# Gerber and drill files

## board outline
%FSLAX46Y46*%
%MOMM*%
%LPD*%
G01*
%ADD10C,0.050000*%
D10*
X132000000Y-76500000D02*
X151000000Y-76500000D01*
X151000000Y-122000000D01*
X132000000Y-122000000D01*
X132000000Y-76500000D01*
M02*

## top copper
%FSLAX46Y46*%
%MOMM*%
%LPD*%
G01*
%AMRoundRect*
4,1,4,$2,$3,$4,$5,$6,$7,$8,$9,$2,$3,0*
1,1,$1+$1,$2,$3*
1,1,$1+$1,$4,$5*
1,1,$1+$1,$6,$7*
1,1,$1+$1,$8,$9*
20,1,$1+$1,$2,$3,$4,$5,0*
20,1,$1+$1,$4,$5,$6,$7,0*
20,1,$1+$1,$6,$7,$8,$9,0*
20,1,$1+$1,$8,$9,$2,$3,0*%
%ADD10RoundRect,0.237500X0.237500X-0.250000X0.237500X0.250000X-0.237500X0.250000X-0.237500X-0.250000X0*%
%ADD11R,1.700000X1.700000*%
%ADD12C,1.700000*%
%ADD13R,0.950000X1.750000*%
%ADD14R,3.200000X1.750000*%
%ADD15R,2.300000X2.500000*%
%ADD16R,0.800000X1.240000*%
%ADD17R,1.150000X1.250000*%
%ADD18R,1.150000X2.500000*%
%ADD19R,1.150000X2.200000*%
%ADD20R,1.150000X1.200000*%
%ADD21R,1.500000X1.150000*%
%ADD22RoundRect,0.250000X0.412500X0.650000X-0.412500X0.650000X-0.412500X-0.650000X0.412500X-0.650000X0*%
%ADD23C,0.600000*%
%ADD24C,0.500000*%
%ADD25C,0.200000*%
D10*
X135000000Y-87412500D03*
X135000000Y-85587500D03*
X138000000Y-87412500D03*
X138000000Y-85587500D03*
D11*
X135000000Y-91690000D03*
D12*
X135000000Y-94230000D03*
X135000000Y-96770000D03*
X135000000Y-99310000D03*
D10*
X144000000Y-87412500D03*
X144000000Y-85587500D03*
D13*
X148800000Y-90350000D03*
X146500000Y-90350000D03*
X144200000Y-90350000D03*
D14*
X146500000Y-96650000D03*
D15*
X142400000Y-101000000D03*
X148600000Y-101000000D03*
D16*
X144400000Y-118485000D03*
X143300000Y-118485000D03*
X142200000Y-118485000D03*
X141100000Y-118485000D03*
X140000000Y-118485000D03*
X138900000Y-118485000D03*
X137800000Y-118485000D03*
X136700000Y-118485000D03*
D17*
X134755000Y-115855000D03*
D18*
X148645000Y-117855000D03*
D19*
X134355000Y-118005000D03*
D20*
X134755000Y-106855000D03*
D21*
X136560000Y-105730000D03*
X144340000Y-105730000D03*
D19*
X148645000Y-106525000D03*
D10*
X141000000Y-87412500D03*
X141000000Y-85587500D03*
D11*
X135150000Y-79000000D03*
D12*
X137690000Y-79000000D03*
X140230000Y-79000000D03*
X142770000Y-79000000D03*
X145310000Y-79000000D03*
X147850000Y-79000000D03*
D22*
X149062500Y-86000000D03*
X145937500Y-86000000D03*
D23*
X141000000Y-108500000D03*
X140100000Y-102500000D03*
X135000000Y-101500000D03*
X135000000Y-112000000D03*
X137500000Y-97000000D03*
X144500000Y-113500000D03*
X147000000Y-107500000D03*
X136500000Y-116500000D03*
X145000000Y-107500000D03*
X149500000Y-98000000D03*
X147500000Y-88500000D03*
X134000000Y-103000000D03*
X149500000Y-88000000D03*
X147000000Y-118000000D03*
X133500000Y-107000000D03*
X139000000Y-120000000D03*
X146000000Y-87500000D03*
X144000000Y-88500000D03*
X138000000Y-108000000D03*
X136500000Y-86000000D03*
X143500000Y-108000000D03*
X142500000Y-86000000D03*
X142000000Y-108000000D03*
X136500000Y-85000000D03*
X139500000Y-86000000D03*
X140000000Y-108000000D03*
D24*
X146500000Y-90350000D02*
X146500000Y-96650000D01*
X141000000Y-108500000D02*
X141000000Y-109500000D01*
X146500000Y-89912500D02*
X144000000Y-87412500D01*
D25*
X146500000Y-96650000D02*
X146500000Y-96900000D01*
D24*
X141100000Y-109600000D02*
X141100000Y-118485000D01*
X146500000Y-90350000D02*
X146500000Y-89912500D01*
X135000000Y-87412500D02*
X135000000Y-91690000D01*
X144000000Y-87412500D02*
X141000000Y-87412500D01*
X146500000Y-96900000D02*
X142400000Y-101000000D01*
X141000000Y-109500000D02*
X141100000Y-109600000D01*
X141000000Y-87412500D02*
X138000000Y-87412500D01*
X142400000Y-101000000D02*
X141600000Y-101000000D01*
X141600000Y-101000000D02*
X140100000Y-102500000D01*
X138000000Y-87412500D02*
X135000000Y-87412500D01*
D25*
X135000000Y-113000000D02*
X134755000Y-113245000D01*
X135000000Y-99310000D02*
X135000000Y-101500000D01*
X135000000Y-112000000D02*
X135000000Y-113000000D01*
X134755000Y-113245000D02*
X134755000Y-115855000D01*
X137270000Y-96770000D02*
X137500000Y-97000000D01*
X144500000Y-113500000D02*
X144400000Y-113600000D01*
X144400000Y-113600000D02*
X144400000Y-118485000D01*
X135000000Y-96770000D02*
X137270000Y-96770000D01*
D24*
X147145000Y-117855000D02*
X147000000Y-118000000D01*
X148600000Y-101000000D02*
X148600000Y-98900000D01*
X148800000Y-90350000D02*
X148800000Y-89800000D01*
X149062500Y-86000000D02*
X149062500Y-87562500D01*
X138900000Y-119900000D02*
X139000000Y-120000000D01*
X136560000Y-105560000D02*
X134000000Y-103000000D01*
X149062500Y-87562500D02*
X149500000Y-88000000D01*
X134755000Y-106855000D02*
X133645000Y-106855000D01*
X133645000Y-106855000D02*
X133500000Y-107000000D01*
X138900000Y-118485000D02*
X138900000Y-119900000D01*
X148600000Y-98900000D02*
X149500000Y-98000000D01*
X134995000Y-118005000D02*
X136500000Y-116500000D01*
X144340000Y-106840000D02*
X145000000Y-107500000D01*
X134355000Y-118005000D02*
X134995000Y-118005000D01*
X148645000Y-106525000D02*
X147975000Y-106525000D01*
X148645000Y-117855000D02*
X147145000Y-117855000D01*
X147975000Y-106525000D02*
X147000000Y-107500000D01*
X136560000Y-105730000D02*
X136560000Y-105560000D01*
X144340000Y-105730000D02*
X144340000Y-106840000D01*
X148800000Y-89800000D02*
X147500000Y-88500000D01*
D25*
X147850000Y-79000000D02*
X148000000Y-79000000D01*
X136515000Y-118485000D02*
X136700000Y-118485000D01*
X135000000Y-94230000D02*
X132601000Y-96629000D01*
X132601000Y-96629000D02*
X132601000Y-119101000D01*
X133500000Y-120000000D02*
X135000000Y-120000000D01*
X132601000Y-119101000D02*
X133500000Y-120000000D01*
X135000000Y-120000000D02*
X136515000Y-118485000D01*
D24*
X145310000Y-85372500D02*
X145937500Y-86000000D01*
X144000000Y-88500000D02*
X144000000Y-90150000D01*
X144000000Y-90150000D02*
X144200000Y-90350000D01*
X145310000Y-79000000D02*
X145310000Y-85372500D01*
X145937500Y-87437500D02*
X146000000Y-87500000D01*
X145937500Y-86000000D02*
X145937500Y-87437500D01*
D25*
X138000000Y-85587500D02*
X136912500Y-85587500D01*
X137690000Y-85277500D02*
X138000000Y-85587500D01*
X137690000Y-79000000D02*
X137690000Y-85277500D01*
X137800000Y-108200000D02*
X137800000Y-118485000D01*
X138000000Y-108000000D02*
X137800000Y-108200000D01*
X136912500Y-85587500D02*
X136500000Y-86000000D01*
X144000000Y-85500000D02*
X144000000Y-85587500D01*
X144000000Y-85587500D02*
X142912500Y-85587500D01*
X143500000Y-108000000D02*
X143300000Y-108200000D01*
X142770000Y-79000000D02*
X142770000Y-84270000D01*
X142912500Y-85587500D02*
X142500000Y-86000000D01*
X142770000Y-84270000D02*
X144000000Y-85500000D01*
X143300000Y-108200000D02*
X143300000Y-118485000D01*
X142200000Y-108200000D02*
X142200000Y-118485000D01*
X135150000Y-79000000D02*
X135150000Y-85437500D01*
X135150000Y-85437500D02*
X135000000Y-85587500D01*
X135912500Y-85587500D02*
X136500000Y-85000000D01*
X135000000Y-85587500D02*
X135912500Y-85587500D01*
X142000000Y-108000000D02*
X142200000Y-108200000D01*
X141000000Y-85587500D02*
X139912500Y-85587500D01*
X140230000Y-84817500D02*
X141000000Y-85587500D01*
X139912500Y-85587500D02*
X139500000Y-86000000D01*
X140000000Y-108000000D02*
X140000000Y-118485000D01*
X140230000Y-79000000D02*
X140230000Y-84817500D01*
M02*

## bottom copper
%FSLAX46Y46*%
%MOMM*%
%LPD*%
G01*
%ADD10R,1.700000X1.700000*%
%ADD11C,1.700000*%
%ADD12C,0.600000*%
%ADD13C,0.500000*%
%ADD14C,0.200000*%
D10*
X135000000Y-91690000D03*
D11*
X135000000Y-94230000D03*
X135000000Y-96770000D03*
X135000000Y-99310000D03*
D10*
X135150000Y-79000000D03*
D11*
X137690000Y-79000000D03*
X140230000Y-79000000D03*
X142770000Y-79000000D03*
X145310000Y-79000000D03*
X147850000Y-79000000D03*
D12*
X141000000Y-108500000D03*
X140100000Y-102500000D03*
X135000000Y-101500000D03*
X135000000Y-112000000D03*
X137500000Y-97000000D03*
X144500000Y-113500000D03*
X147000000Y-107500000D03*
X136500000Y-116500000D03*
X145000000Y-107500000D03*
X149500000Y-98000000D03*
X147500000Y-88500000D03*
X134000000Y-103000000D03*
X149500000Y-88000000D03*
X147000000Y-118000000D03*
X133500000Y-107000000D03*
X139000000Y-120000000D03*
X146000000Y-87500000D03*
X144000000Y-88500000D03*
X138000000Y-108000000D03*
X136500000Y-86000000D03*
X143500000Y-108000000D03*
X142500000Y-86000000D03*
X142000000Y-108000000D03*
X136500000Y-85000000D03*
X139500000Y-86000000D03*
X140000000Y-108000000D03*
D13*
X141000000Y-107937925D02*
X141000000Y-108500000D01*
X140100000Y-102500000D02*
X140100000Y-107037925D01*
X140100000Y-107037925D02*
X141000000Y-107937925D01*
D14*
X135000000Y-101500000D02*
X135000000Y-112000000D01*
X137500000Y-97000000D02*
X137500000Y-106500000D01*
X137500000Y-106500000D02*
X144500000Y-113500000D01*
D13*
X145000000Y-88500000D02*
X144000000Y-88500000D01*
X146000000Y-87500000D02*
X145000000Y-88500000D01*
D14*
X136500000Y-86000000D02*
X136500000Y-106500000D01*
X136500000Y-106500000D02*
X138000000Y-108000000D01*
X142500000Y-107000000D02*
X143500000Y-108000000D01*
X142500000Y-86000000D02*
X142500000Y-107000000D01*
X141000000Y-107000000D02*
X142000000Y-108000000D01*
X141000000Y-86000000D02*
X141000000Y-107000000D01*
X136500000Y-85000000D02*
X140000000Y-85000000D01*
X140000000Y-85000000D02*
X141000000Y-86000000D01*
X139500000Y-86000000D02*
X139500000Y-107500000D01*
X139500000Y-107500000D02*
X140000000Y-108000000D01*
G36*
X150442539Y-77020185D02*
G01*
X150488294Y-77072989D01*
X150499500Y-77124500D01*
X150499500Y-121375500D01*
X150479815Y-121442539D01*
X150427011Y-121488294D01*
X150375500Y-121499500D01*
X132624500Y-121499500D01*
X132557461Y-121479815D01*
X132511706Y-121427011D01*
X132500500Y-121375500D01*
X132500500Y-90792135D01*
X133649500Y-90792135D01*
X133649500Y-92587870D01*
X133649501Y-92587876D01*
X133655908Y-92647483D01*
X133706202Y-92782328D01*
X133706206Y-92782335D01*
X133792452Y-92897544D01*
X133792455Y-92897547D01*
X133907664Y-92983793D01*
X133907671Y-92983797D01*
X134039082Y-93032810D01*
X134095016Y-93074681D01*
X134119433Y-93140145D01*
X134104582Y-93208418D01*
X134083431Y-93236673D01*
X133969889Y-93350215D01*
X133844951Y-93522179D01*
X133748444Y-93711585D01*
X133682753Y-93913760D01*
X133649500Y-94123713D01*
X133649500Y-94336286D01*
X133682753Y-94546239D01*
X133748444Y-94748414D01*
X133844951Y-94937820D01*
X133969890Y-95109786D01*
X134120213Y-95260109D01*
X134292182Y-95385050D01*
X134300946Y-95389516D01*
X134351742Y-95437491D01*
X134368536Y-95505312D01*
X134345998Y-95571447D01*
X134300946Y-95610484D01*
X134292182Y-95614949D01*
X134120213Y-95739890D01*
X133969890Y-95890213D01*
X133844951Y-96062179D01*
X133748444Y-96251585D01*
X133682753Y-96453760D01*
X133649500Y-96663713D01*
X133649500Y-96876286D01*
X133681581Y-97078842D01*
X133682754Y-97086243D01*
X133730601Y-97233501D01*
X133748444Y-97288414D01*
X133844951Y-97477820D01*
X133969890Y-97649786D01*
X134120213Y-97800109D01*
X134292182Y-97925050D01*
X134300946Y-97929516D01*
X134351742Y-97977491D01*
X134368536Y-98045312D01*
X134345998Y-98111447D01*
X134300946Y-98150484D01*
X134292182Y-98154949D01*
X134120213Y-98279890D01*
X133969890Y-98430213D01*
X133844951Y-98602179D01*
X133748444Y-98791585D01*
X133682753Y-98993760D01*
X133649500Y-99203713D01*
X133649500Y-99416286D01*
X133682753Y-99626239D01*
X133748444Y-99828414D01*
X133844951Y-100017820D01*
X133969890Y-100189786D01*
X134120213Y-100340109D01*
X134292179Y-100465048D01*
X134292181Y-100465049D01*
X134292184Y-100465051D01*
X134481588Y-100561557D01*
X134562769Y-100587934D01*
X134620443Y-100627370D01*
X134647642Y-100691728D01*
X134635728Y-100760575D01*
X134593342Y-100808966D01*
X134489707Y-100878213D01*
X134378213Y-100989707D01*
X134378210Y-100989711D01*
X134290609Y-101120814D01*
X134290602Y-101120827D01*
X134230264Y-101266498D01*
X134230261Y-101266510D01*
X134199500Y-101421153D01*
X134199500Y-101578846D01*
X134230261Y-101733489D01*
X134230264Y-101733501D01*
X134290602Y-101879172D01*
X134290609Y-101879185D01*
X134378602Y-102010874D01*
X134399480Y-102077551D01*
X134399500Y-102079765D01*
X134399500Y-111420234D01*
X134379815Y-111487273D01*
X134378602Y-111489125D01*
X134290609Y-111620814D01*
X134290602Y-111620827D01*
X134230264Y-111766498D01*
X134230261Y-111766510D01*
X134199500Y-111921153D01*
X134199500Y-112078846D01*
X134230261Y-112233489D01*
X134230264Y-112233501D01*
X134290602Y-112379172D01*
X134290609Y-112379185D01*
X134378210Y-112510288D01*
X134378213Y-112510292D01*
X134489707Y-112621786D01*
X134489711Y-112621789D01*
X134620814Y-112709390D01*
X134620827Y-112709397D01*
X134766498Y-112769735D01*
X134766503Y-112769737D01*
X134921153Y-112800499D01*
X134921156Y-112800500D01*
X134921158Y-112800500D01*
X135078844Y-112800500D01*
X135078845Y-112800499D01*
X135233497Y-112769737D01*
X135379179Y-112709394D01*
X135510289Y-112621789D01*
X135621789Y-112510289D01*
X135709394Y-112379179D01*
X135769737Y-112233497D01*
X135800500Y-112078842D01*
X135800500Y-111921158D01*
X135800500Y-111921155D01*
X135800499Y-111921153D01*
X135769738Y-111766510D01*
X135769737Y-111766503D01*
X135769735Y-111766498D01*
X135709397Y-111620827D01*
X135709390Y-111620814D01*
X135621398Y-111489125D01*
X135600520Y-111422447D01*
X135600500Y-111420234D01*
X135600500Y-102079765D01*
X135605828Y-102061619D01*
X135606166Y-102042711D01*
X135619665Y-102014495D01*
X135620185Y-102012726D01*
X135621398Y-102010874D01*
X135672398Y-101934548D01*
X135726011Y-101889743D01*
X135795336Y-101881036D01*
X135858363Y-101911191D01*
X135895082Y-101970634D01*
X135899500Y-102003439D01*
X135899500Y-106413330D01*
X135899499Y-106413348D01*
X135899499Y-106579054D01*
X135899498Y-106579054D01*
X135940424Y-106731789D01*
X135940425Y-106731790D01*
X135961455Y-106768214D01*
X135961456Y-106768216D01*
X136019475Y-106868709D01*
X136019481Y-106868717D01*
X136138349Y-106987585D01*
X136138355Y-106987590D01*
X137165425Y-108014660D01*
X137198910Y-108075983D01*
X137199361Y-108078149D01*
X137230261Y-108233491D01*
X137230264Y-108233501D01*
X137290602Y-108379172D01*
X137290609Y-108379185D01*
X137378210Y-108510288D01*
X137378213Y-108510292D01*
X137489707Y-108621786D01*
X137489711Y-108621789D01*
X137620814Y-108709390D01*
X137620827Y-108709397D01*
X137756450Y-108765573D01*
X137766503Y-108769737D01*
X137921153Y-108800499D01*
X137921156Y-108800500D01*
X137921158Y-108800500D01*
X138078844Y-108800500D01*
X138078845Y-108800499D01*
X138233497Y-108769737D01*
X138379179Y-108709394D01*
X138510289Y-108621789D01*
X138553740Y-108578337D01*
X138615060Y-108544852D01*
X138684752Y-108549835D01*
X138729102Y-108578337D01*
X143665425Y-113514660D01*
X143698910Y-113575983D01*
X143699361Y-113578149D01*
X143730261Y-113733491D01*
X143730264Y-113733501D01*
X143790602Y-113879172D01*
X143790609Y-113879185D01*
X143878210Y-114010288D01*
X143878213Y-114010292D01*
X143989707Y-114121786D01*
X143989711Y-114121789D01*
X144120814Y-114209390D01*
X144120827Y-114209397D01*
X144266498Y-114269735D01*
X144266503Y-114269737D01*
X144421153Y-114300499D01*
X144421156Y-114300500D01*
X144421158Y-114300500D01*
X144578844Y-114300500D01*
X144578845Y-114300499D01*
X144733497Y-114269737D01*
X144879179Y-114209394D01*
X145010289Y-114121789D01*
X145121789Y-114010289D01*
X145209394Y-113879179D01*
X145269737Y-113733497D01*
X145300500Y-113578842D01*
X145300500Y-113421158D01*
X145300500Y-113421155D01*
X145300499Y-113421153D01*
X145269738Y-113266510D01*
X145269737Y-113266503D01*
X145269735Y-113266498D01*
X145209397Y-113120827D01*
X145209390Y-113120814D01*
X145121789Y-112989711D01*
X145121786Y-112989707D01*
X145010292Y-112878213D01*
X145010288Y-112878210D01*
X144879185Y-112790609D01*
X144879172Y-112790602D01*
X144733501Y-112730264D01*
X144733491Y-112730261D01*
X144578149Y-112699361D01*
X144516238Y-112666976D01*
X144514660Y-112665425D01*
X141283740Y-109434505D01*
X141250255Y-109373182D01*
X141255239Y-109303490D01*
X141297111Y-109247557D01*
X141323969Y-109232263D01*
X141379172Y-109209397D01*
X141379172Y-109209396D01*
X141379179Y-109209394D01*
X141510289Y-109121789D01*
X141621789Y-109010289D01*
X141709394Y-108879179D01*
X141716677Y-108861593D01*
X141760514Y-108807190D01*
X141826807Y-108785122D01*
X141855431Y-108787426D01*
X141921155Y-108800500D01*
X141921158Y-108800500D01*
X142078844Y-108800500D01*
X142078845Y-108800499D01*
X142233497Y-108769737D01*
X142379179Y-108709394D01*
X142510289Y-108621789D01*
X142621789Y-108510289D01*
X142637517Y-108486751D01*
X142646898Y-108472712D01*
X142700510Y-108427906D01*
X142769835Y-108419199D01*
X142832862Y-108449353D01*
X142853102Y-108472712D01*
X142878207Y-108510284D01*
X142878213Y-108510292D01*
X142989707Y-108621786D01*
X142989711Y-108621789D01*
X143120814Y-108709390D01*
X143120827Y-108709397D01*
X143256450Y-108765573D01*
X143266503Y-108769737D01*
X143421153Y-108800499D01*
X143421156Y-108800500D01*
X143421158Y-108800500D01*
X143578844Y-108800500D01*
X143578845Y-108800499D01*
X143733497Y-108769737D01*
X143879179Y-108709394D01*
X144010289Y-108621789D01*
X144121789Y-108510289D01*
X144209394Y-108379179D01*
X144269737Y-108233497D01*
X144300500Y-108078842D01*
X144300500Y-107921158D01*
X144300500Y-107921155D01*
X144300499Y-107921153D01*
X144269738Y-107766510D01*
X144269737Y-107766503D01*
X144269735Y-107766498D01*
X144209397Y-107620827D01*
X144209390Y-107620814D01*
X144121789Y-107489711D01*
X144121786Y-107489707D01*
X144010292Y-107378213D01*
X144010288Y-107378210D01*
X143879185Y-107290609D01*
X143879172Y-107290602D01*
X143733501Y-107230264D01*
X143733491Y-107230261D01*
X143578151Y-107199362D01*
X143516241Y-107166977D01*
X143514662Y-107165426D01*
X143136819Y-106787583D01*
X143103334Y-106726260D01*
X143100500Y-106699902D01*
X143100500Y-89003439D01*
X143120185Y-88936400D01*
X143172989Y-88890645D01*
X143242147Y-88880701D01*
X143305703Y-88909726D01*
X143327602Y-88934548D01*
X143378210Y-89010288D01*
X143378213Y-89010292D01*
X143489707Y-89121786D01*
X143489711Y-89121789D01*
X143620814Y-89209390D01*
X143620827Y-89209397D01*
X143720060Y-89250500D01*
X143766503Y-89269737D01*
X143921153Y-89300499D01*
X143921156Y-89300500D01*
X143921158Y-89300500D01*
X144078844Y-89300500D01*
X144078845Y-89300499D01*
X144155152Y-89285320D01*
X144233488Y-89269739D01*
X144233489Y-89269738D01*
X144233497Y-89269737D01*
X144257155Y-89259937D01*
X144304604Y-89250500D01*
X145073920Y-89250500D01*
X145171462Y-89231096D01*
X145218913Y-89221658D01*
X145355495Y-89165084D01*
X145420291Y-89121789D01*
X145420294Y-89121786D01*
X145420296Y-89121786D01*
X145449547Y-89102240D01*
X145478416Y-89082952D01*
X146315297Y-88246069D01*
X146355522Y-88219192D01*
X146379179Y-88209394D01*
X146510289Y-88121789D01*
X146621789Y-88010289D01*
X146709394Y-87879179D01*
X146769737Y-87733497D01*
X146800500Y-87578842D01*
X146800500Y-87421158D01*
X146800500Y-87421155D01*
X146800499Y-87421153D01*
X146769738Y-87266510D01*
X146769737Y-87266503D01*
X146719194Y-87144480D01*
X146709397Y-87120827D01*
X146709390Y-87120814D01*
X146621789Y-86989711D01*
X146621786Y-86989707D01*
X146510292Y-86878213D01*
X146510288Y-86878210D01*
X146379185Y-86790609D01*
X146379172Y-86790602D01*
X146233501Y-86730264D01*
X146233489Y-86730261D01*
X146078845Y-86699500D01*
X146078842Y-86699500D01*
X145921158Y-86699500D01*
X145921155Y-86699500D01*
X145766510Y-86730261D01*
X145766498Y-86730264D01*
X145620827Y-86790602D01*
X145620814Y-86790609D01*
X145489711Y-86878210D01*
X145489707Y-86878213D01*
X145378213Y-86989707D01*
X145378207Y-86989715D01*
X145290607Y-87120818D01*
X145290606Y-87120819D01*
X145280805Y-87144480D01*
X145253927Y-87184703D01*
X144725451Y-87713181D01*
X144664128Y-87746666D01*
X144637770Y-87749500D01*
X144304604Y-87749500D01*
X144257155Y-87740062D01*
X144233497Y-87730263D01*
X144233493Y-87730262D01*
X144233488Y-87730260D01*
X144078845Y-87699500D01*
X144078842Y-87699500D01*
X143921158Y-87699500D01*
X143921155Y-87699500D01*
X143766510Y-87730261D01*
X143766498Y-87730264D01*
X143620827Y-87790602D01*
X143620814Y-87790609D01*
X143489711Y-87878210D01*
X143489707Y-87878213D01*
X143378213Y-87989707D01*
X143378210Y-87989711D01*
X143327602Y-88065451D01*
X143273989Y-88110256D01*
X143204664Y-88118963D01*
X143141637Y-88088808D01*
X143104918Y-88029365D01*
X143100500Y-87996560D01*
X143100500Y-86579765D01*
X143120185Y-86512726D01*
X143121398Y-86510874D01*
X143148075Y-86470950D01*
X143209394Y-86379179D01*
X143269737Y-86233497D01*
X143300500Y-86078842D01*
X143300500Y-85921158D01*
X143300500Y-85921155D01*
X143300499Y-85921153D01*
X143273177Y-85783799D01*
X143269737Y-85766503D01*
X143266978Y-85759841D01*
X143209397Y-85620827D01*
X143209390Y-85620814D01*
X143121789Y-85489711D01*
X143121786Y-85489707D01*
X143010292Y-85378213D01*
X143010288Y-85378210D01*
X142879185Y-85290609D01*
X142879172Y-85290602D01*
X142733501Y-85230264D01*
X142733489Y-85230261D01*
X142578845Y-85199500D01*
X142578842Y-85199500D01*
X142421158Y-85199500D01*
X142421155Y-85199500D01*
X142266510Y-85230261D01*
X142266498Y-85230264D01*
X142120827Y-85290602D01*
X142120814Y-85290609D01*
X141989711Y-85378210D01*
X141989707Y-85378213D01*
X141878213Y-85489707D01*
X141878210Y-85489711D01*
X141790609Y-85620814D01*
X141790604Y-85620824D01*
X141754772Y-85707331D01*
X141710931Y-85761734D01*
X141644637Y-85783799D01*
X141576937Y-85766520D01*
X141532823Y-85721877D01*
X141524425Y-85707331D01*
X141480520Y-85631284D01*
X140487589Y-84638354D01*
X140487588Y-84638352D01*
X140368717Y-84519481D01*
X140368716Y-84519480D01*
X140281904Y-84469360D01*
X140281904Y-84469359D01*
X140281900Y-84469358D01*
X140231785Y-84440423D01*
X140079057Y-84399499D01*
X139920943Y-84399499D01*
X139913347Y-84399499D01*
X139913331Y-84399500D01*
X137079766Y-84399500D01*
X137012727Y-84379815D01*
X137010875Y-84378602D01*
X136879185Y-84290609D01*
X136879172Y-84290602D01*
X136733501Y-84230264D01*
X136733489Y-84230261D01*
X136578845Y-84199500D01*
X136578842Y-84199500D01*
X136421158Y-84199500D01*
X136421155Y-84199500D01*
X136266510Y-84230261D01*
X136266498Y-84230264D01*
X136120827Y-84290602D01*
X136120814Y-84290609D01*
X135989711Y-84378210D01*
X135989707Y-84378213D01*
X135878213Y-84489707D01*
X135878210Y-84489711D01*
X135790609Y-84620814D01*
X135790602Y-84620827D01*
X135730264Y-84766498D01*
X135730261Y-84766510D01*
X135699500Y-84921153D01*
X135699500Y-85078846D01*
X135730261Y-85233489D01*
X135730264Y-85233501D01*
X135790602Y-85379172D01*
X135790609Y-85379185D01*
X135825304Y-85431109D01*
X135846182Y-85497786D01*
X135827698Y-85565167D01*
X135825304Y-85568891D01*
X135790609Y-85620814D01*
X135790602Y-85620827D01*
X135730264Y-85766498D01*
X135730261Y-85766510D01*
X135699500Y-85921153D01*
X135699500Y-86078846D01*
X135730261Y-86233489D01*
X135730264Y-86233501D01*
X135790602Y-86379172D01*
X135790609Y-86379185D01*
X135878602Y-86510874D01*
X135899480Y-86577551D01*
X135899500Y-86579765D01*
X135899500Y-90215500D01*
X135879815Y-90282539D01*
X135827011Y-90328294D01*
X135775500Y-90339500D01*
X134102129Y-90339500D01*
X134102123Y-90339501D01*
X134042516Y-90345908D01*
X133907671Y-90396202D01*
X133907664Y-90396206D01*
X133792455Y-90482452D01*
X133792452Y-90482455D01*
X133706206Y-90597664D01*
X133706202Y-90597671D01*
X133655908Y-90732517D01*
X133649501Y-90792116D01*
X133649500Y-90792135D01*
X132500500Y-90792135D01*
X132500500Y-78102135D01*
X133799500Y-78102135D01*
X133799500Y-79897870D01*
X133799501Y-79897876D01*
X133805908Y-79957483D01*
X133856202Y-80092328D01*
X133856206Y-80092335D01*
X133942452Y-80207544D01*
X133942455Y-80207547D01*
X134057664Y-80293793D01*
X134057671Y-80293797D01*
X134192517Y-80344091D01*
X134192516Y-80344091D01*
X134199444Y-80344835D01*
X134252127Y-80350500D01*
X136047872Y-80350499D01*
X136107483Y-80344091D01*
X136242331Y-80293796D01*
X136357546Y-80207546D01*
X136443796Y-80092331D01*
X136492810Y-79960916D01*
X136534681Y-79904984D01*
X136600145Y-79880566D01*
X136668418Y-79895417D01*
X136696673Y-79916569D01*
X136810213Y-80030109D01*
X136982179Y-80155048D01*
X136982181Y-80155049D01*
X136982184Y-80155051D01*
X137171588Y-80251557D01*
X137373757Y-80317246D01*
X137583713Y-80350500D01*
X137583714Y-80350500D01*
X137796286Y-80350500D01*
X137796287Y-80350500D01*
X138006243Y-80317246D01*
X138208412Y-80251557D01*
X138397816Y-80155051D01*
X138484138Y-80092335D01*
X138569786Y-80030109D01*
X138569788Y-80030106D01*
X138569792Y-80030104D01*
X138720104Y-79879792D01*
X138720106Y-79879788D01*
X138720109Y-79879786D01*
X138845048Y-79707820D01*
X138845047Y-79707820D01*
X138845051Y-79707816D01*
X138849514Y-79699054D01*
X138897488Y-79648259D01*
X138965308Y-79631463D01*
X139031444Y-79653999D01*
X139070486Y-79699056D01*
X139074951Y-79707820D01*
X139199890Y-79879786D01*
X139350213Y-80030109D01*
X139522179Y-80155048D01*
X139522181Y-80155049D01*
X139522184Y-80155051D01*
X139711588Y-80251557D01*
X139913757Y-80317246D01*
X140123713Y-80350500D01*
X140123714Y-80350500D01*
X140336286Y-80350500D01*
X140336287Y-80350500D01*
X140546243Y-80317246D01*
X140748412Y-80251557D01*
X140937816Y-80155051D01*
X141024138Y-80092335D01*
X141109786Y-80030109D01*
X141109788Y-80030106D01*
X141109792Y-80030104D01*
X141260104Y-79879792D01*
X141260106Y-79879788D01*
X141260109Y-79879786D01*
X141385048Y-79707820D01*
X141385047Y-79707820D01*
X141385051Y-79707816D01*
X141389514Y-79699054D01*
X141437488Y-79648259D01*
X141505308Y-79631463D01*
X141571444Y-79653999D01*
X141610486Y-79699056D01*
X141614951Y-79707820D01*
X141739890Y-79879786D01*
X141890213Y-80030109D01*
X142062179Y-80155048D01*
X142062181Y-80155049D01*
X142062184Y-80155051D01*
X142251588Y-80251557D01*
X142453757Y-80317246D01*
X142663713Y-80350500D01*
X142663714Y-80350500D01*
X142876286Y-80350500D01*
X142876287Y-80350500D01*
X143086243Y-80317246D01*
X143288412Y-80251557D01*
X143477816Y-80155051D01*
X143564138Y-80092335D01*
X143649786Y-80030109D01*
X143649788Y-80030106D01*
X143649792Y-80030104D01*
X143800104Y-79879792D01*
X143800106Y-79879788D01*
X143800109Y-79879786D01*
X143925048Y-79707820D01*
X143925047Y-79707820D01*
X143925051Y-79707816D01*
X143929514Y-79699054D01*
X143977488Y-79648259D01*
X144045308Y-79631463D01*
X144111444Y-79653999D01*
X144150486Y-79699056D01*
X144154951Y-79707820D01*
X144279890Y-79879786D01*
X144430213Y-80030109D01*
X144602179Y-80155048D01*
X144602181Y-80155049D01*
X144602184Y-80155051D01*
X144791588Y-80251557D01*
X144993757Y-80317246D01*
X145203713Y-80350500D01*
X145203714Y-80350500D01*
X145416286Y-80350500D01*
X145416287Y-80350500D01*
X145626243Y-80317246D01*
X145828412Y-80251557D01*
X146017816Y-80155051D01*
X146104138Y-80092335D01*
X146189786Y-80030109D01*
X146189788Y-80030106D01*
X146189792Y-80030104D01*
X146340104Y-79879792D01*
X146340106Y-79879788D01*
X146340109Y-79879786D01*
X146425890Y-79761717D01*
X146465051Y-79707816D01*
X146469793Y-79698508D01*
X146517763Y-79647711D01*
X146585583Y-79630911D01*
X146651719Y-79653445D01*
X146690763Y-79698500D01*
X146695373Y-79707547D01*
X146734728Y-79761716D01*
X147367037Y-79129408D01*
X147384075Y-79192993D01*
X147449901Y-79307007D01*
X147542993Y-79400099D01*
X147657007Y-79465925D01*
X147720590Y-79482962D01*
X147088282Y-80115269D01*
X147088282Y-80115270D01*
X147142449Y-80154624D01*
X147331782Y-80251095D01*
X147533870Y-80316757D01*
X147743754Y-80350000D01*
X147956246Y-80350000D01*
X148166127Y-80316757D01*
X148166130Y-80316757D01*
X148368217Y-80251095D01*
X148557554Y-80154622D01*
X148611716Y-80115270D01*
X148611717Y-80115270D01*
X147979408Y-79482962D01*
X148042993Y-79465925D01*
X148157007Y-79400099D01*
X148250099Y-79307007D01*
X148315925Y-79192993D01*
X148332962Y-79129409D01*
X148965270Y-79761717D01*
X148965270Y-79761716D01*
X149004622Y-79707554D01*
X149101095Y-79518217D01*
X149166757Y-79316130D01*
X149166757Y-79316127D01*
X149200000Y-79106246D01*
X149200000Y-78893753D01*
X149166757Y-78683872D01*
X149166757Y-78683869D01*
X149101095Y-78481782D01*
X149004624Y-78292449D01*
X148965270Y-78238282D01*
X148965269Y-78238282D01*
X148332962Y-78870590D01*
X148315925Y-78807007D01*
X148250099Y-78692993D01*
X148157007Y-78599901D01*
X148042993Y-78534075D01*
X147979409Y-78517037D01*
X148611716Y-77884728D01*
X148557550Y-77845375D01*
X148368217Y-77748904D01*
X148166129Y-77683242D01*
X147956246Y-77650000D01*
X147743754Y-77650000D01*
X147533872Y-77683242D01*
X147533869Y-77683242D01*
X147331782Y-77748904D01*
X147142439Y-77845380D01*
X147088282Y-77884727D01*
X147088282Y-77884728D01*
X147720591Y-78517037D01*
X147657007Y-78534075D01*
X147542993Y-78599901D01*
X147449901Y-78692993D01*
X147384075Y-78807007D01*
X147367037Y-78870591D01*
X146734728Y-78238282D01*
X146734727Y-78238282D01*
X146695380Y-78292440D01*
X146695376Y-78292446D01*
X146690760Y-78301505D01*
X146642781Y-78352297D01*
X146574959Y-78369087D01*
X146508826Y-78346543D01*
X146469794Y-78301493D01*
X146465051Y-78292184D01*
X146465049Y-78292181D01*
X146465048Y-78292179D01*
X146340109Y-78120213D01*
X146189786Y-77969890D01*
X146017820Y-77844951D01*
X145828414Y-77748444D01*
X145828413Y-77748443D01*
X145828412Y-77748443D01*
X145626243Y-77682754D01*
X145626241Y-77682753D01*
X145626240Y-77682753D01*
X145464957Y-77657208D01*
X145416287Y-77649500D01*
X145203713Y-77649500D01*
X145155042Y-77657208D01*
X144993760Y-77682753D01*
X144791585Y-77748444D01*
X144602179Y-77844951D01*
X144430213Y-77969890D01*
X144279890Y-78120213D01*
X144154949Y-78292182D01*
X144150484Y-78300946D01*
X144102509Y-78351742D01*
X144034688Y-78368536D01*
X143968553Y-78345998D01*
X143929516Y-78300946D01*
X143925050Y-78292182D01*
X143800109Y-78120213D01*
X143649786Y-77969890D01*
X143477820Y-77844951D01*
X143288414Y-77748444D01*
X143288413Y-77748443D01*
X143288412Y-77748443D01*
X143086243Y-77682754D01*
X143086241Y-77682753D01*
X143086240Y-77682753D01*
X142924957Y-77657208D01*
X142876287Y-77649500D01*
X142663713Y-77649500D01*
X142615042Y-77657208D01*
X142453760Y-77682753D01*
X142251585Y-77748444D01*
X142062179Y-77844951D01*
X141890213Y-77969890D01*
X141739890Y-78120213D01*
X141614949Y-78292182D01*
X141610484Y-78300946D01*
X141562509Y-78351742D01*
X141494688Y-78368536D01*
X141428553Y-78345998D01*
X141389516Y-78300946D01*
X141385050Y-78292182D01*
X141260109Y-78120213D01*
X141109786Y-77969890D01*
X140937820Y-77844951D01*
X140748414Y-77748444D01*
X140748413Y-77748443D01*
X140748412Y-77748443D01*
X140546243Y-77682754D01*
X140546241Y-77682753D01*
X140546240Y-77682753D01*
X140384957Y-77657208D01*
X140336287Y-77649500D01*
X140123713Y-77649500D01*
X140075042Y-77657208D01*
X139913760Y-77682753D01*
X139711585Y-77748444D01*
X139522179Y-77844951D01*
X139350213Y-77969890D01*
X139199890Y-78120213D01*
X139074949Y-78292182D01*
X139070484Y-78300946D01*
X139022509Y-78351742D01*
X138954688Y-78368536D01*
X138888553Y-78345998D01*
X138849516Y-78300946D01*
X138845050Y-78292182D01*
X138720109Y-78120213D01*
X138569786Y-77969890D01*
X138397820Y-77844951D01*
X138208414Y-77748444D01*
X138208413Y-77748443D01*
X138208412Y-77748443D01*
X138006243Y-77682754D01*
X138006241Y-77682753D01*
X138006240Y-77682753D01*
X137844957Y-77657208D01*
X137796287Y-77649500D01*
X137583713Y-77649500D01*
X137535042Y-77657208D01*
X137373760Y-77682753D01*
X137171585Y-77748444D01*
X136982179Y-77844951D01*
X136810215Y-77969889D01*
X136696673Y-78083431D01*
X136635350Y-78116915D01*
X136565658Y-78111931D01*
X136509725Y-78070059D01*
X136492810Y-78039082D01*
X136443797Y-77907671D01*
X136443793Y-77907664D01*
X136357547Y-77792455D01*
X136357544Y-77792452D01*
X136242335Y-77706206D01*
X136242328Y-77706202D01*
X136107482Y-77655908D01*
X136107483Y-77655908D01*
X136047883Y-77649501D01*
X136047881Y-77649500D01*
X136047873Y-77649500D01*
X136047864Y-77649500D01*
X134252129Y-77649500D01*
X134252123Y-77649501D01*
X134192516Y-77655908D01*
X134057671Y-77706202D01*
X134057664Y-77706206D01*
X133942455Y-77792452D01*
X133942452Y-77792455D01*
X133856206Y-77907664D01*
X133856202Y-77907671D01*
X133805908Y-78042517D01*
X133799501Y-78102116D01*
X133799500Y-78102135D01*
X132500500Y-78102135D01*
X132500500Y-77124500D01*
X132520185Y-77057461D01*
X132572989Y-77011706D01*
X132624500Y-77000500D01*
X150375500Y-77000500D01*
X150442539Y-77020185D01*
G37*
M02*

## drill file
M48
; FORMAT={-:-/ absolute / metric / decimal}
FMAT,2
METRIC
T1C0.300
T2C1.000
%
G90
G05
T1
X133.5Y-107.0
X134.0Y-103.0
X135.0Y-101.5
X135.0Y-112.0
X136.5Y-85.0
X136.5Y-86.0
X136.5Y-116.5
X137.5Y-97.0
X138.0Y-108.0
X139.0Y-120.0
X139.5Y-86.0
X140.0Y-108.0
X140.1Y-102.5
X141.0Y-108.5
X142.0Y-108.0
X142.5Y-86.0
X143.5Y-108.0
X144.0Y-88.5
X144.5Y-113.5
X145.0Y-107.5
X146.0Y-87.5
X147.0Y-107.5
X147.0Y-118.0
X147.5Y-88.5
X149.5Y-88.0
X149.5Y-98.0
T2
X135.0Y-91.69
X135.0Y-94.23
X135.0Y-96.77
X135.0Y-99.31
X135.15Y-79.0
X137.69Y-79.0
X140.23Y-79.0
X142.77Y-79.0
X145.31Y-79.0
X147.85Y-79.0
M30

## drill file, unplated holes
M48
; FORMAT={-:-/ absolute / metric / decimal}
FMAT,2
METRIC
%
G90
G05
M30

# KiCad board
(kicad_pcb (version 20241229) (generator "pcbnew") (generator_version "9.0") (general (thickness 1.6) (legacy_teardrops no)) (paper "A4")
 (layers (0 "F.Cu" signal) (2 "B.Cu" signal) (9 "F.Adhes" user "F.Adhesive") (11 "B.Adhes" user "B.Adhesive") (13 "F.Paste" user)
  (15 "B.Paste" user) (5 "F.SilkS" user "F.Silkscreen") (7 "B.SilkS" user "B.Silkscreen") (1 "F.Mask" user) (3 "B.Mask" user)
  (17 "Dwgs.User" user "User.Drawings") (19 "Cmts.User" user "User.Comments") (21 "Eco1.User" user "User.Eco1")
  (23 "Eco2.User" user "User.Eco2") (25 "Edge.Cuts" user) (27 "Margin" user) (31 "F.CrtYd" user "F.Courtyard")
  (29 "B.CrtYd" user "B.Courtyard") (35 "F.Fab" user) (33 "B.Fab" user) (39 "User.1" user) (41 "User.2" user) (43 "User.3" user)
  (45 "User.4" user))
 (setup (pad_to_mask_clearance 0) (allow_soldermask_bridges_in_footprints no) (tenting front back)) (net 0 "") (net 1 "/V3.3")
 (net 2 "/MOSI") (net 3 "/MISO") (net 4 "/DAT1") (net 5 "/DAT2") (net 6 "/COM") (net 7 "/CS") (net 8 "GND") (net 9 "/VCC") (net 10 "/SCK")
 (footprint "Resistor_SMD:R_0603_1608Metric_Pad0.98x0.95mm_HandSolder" (layer "F.Cu") (at 135 86.5 90)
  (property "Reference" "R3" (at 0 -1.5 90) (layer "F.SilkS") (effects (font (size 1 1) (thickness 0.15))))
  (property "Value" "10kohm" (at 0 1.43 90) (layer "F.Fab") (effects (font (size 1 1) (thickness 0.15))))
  (pad "1" smd roundrect (at -0.9125 0 90) (size 0.975 0.95) (layers "F.Cu" "F.Mask" "F.Paste") (roundrect_rratio 0.25) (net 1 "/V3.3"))
  (pad "2" smd roundrect (at 0.9125 0 90) (size 0.975 0.95) (layers "F.Cu" "F.Mask" "F.Paste") (roundrect_rratio 0.25) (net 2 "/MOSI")))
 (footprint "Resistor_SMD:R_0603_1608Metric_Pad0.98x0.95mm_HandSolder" (layer "F.Cu") (at 138 86.5 90)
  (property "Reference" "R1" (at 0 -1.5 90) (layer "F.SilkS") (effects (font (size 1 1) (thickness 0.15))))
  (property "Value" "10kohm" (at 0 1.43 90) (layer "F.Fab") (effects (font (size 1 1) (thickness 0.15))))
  (pad "1" smd roundrect (at -0.9125 0 90) (size 0.975 0.95) (layers "F.Cu" "F.Mask" "F.Paste") (roundrect_rratio 0.25) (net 1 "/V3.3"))
  (pad "2" smd roundrect (at 0.9125 0 90) (size 0.975 0.95) (layers "F.Cu" "F.Mask" "F.Paste") (roundrect_rratio 0.25) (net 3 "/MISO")))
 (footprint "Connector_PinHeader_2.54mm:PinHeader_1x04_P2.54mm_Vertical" (layer "F.Cu") (at 135 91.69)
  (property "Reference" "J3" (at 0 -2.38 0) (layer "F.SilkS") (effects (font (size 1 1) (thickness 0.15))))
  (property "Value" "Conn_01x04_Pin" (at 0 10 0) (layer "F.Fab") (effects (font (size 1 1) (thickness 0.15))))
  (pad "1" thru_hole rect (at 0 0) (size 1.7 1.7) (drill 1) (layers "*.Cu" "*.Mask") (remove_unused_layers no) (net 1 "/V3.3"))
  (pad "2" thru_hole circle (at 0 2.54) (size 1.7 1.7) (drill 1) (layers "*.Cu" "*.Mask") (remove_unused_layers no) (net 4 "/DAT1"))
  (pad "3" thru_hole circle (at 0 5.08) (size 1.7 1.7) (drill 1) (layers "*.Cu" "*.Mask") (remove_unused_layers no) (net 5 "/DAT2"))
  (pad "4" thru_hole circle (at 0 7.62) (size 1.7 1.7) (drill 1) (layers "*.Cu" "*.Mask") (remove_unused_layers no) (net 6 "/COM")))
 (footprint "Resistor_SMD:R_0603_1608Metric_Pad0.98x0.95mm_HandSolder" (layer "F.Cu") (at 144 86.5 90)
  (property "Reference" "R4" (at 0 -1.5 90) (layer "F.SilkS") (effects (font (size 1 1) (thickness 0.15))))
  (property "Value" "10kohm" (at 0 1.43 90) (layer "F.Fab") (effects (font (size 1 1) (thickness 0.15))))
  (pad "1" smd roundrect (at -0.9125 0 90) (size 0.975 0.95) (layers "F.Cu" "F.Mask" "F.Paste") (roundrect_rratio 0.25) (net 1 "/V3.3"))
  (pad "2" smd roundrect (at 0.9125 0 90) (size 0.975 0.95) (layers "F.Cu" "F.Mask" "F.Paste") (roundrect_rratio 0.25) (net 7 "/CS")))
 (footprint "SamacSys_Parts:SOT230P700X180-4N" (layer "F.Cu") (at 146.5 93.5 -90)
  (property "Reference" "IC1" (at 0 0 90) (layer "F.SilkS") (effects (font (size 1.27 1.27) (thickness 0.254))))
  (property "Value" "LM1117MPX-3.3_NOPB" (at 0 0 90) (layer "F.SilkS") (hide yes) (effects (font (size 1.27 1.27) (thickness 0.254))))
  (pad "1" smd rect (at -3.15 -2.3) (size 0.95 1.75) (layers "F.Cu" "F.Mask" "F.Paste") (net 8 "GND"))
  (pad "2" smd rect (at -3.15 0) (size 0.95 1.75) (layers "F.Cu" "F.Mask" "F.Paste") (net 1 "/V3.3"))
  (pad "3" smd rect (at -3.15 2.3) (size 0.95 1.75) (layers "F.Cu" "F.Mask" "F.Paste") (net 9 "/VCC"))
  (pad "4" smd rect (at 3.15 0 270) (size 1.75 3.2) (layers "F.Cu" "F.Mask" "F.Paste") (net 1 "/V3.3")))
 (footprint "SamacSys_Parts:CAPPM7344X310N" (layer "F.Cu") (at 145.5 101)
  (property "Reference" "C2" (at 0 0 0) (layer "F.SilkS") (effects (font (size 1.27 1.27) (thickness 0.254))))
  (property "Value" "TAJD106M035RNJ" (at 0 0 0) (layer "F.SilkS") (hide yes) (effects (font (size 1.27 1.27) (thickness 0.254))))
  (pad "1" smd rect (at -3.1 0) (size 2.3 2.5) (layers "F.Cu" "F.Mask" "F.Paste") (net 1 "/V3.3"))
  (pad "2" smd rect (at 3.1 0) (size 2.3 2.5) (layers "F.Cu" "F.Mask" "F.Paste") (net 8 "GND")))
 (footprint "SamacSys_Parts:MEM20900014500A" (layer "F.Cu") (at 141.5 112.5)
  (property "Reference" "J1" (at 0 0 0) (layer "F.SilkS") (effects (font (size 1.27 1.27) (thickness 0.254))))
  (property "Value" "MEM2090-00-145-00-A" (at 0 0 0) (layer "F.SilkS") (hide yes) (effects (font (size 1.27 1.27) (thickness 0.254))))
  (pad "1" smd rect (at 2.9 5.985) (size 0.8 1.24) (layers "F.Cu" "F.Mask" "F.Paste") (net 5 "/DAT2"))
  (pad "2" smd rect (at 1.8 5.985) (size 0.8 1.24) (layers "F.Cu" "F.Mask" "F.Paste") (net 7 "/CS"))
  (pad "3" smd rect (at 0.7 5.985) (size 0.8 1.24) (layers "F.Cu" "F.Mask" "F.Paste") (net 2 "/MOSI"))
  (pad "4" smd rect (at -0.4 5.985) (size 0.8 1.24) (layers "F.Cu" "F.Mask" "F.Paste") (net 1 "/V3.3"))
  (pad "5" smd rect (at -1.5 5.985) (size 0.8 1.24) (layers "F.Cu" "F.Mask" "F.Paste") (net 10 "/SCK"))
  (pad "6" smd rect (at -2.6 5.985) (size 0.8 1.24) (layers "F.Cu" "F.Mask" "F.Paste") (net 8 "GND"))
  (pad "7" smd rect (at -3.7 5.985) (size 0.8 1.24) (layers "F.Cu" "F.Mask" "F.Paste") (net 3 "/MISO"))
  (pad "8" smd rect (at -4.8 5.985) (size 0.8 1.24) (layers "F.Cu" "F.Mask" "F.Paste") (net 4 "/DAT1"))
  (pad "9" smd rect (at -6.745 3.355) (size 1.15 1.25) (layers "F.Cu" "F.Mask" "F.Paste") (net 6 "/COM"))
  (pad "10" smd rect (at 7.145 5.355) (size 1.15 2.5) (layers "F.Cu" "F.Mask" "F.Paste") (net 8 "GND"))
  (pad "11" smd rect (at -7.145 5.505) (size 1.15 2.2) (layers "F.Cu" "F.Mask" "F.Paste") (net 8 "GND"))
  (pad "12" smd rect (at -6.745 -5.645) (size 1.15 1.2) (layers "F.Cu" "F.Mask" "F.Paste") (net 8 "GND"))
  (pad "13" smd rect (at -4.94 -6.77 90) (size 1.15 1.5) (layers "F.Cu" "F.Mask" "F.Paste") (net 8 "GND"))
  (pad "14" smd rect (at 2.84 -6.77 90) (size 1.15 1.5) (layers "F.Cu" "F.Mask" "F.Paste") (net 8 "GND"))
  (pad "15" smd rect (at 7.145 -5.975) (size 1.15 2.2) (layers "F.Cu" "F.Mask" "F.Paste") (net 8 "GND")))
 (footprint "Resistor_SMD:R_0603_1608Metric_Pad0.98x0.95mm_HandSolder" (layer "F.Cu") (at 141 86.5 90)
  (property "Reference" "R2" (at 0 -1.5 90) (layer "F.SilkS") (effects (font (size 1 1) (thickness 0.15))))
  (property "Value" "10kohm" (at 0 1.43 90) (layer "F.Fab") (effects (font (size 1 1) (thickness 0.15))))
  (pad "1" smd roundrect (at -0.9125 0 90) (size 0.975 0.95) (layers "F.Cu" "F.Mask" "F.Paste") (roundrect_rratio 0.25) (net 1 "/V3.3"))
  (pad "2" smd roundrect (at 0.9125 0 90) (size 0.975 0.95) (layers "F.Cu" "F.Mask" "F.Paste") (roundrect_rratio 0.25) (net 10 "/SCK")))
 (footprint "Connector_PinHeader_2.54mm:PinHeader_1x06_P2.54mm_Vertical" (layer "F.Cu") (at 135.15 79 90)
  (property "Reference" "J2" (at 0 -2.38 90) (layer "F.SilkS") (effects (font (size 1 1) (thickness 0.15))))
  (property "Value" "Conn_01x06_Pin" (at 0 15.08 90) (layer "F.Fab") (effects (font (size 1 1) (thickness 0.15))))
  (pad "1" thru_hole rect (at 0 0 90) (size 1.7 1.7) (drill 1) (layers "*.Cu" "*.Mask") (remove_unused_layers no) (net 2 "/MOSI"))
  (pad "2" thru_hole circle (at 0 2.54 90) (size 1.7 1.7) (drill 1) (layers "*.Cu" "*.Mask") (remove_unused_layers no) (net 3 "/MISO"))
  (pad "3" thru_hole circle (at 0 5.08 90) (size 1.7 1.7) (drill 1) (layers "*.Cu" "*.Mask") (remove_unused_layers no) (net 10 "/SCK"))
  (pad "4" thru_hole circle (at 0 7.62 90) (size 1.7 1.7) (drill 1) (layers "*.Cu" "*.Mask") (remove_unused_layers no) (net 7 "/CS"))
  (pad "5" thru_hole circle (at 0 10.16 90) (size 1.7 1.7) (drill 1) (layers "*.Cu" "*.Mask") (remove_unused_layers no) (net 9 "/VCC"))
  (pad "6" thru_hole circle (at 0 12.7 90) (size 1.7 1.7) (drill 1) (layers "*.Cu" "*.Mask") (remove_unused_layers no) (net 8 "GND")))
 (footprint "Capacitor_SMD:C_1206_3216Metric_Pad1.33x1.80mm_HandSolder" (layer "F.Cu") (at 147.5 86 180)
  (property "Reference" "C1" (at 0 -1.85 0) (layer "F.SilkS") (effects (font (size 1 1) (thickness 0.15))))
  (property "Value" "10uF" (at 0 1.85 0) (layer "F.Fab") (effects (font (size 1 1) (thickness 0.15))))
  (pad "1" smd roundrect (at -1.5625 0 180) (size 1.325 1.8) (layers "F.Cu" "F.Mask" "F.Paste") (roundrect_rratio 0.188679) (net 8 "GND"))
  (pad "2" smd roundrect (at 1.5625 0 180) (size 1.325 1.8) (layers "F.Cu" "F.Mask" "F.Paste") (roundrect_rratio 0.188679) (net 9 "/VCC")))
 (gr_rect (start 132 76.5) (end 151 122) (stroke (width 0.05) (type default)) (fill no) (layer "Edge.Cuts"))
 (segment (start 146.5 90.35) (end 146.5 96.65) (width 0.5) (layer "F.Cu") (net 1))
 (segment (start 141 108.5) (end 141 109.5) (width 0.5) (layer "F.Cu") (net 1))
 (segment (start 146.5 89.9125) (end 144 87.4125) (width 0.5) (layer "F.Cu") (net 1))
 (segment (start 146.5 96.65) (end 146.5 96.9) (width 0.2) (layer "F.Cu") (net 1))
 (segment (start 141.1 109.6) (end 141.1 118.485) (width 0.5) (layer "F.Cu") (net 1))
 (segment (start 146.5 90.35) (end 146.5 89.9125) (width 0.5) (layer "F.Cu") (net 1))
 (segment (start 135 87.4125) (end 135 91.69) (width 0.5) (layer "F.Cu") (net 1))
 (segment (start 144 87.4125) (end 141 87.4125) (width 0.5) (layer "F.Cu") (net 1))
 (segment (start 146.5 96.9) (end 142.4 101) (width 0.5) (layer "F.Cu") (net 1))
 (segment (start 141 109.5) (end 141.1 109.6) (width 0.5) (layer "F.Cu") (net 1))
 (segment (start 141 87.4125) (end 138 87.4125) (width 0.5) (layer "F.Cu") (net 1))
 (segment (start 142.4 101) (end 141.6 101) (width 0.5) (layer "F.Cu") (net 1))
 (segment (start 141.6 101) (end 140.1 102.5) (width 0.5) (layer "F.Cu") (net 1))
 (segment (start 138 87.4125) (end 135 87.4125) (width 0.5) (layer "F.Cu") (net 1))
 (via (at 141 108.5) (size 0.6) (drill 0.3) (layers "F.Cu" "B.Cu") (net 1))
 (via (at 140.1 102.5) (size 0.6) (drill 0.3) (layers "F.Cu" "B.Cu") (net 1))
 (segment (start 141 107.937925) (end 141 108.5) (width 0.5) (layer "B.Cu") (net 1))
 (segment (start 140.1 102.5) (end 140.1 107.037925) (width 0.5) (layer "B.Cu") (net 1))
 (segment (start 140.1 107.037925) (end 141 107.937925) (width 0.5) (layer "B.Cu") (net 1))
 (segment (start 135 113) (end 134.755 113.245) (width 0.2) (layer "F.Cu") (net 6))
 (segment (start 135 99.31) (end 135 101.5) (width 0.2) (layer "F.Cu") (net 6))
 (segment (start 135 112) (end 135 113) (width 0.2) (layer "F.Cu") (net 6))
 (segment (start 134.755 113.245) (end 134.755 115.855) (width 0.2) (layer "F.Cu") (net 6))
 (via (at 135 101.5) (size 0.6) (drill 0.3) (layers "F.Cu" "B.Cu") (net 6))
 (via (at 135 112) (size 0.6) (drill 0.3) (layers "F.Cu" "B.Cu") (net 6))
 (segment (start 135 101.5) (end 135 112) (width 0.2) (layer "B.Cu") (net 6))
 (segment (start 137.27 96.77) (end 137.5 97) (width 0.2) (layer "F.Cu") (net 5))
 (segment (start 144.5 113.5) (end 144.4 113.6) (width 0.2) (layer "F.Cu") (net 5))
 (segment (start 144.4 113.6) (end 144.4 118.485) (width 0.2) (layer "F.Cu") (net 5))
 (segment (start 135 96.77) (end 137.27 96.77) (width 0.2) (layer "F.Cu") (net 5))
 (via (at 137.5 97) (size 0.6) (drill 0.3) (layers "F.Cu" "B.Cu") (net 5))
 (via (at 144.5 113.5) (size 0.6) (drill 0.3) (layers "F.Cu" "B.Cu") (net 5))
 (segment (start 137.5 97) (end 137.5 106.5) (width 0.2) (layer "B.Cu") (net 5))
 (segment (start 137.5 106.5) (end 144.5 113.5) (width 0.2) (layer "B.Cu") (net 5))
 (segment (start 147.145 117.855) (end 147 118) (width 0.5) (layer "F.Cu") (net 8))
 (segment (start 148.6 101) (end 148.6 98.9) (width 0.5) (layer "F.Cu") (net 8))
 (segment (start 148.8 90.35) (end 148.8 89.8) (width 0.5) (layer "F.Cu") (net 8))
 (segment (start 149.0625 86) (end 149.0625 87.5625) (width 0.5) (layer "F.Cu") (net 8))
 (segment (start 138.9 119.9) (end 139 120) (width 0.5) (layer "F.Cu") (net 8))
 (segment (start 136.56 105.56) (end 134 103) (width 0.5) (layer "F.Cu") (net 8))
 (segment (start 149.0625 87.5625) (end 149.5 88) (width 0.5) (layer "F.Cu") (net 8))
 (segment (start 134.755 106.855) (end 133.645 106.855) (width 0.5) (layer "F.Cu") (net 8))
 (segment (start 133.645 106.855) (end 133.5 107) (width 0.5) (layer "F.Cu") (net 8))
 (segment (start 138.9 118.485) (end 138.9 119.9) (width 0.5) (layer "F.Cu") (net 8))
 (segment (start 148.6 98.9) (end 149.5 98) (width 0.5) (layer "F.Cu") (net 8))
 (segment (start 134.995 118.005) (end 136.5 116.5) (width 0.5) (layer "F.Cu") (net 8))
 (segment (start 144.34 106.84) (end 145 107.5) (width 0.5) (layer "F.Cu") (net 8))
 (segment (start 134.355 118.005) (end 134.995 118.005) (width 0.5) (layer "F.Cu") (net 8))
 (segment (start 148.645 106.525) (end 147.975 106.525) (width 0.5) (layer "F.Cu") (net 8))
 (segment (start 148.645 117.855) (end 147.145 117.855) (width 0.5) (layer "F.Cu") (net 8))
 (segment (start 147.975 106.525) (end 147 107.5) (width 0.5) (layer "F.Cu") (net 8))
 (segment (start 136.56 105.73) (end 136.56 105.56) (width 0.5) (layer "F.Cu") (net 8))
 (segment (start 144.34 105.73) (end 144.34 106.84) (width 0.5) (layer "F.Cu") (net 8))
 (segment (start 148.8 89.8) (end 147.5 88.5) (width 0.5) (layer "F.Cu") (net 8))
 (segment (start 147.85 79) (end 148 79) (width 0.2) (layer "F.Cu") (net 8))
 (via (at 147 107.5) (size 0.6) (drill 0.3) (layers "F.Cu" "B.Cu") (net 8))
 (via (at 136.5 116.5) (size 0.6) (drill 0.3) (layers "F.Cu" "B.Cu") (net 8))
 (via (at 145 107.5) (size 0.6) (drill 0.3) (layers "F.Cu" "B.Cu") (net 8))
 (via (at 149.5 98) (size 0.6) (drill 0.3) (layers "F.Cu" "B.Cu") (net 8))
 (via (at 147.5 88.5) (size 0.6) (drill 0.3) (layers "F.Cu" "B.Cu") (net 8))
 (via (at 134 103) (size 0.6) (drill 0.3) (layers "F.Cu" "B.Cu") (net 8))
 (via (at 149.5 88) (size 0.6) (drill 0.3) (layers "F.Cu" "B.Cu") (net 8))
 (via (at 147 118) (size 0.6) (drill 0.3) (layers "F.Cu" "B.Cu") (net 8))
 (via (at 133.5 107) (size 0.6) (drill 0.3) (layers "F.Cu" "B.Cu") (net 8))
 (via (at 139 120) (size 0.6) (drill 0.3) (layers "F.Cu" "B.Cu") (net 8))
 (segment (start 136.515 118.485) (end 136.7 118.485) (width 0.2) (layer "F.Cu") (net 4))
 (segment (start 135 94.23) (end 132.601 96.629) (width 0.2) (layer "F.Cu") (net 4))
 (segment (start 132.601 96.629) (end 132.601 119.101) (width 0.2) (layer "F.Cu") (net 4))
 (segment (start 133.5 120) (end 135 120) (width 0.2) (layer "F.Cu") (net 4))
 (segment (start 132.601 119.101) (end 133.5 120) (width 0.2) (layer "F.Cu") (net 4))
 (segment (start 135 120) (end 136.515 118.485) (width 0.2) (layer "F.Cu") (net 4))
 (segment (start 145.31 85.3725) (end 145.9375 86) (width 0.5) (layer "F.Cu") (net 9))
 (segment (start 144 88.5) (end 144 90.15) (width 0.5) (layer "F.Cu") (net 9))
 (segment (start 144 90.15) (end 144.2 90.35) (width 0.5) (layer "F.Cu") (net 9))
 (segment (start 145.31 79) (end 145.31 85.3725) (width 0.5) (layer "F.Cu") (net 9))
 (segment (start 145.9375 87.4375) (end 146 87.5) (width 0.5) (layer "F.Cu") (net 9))
 (segment (start 145.9375 86) (end 145.9375 87.4375) (width 0.5) (layer "F.Cu") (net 9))
 (via (at 146 87.5) (size 0.6) (drill 0.3) (layers "F.Cu" "B.Cu") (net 9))
 (via (at 144 88.5) (size 0.6) (drill 0.3) (layers "F.Cu" "B.Cu") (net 9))
 (segment (start 145 88.5) (end 144 88.5) (width 0.5) (layer "B.Cu") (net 9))
 (segment (start 146 87.5) (end 145 88.5) (width 0.5) (layer "B.Cu") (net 9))
 (segment (start 138 85.5875) (end 136.9125 85.5875) (width 0.2) (layer "F.Cu") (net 3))
 (segment (start 137.69 85.2775) (end 138 85.5875) (width 0.2) (layer "F.Cu") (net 3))
 (segment (start 137.69 79) (end 137.69 85.2775) (width 0.2) (layer "F.Cu") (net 3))
 (segment (start 137.8 108.2) (end 137.8 118.485) (width 0.2) (layer "F.Cu") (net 3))
 (segment (start 138 108) (end 137.8 108.2) (width 0.2) (layer "F.Cu") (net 3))
 (segment (start 136.9125 85.5875) (end 136.5 86) (width 0.2) (layer "F.Cu") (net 3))
 (via (at 138 108) (size 0.6) (drill 0.3) (layers "F.Cu" "B.Cu") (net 3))
 (via (at 136.5 86) (size 0.6) (drill 0.3) (layers "F.Cu" "B.Cu") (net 3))
 (segment (start 136.5 86) (end 136.5 106.5) (width 0.2) (layer "B.Cu") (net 3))
 (segment (start 136.5 106.5) (end 138 108) (width 0.2) (layer "B.Cu") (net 3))
 (segment (start 144 85.5) (end 144 85.5875) (width 0.2) (layer "F.Cu") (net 7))
 (segment (start 144 85.5875) (end 142.9125 85.5875) (width 0.2) (layer "F.Cu") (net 7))
 (segment (start 143.5 108) (end 143.3 108.2) (width 0.2) (layer "F.Cu") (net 7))
 (segment (start 142.77 79) (end 142.77 84.27) (width 0.2) (layer "F.Cu") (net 7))
 (segment (start 142.9125 85.5875) (end 142.5 86) (width 0.2) (layer "F.Cu") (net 7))
 (segment (start 142.77 84.27) (end 144 85.5) (width 0.2) (layer "F.Cu") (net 7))
 (segment (start 143.3 108.2) (end 143.3 118.485) (width 0.2) (layer "F.Cu") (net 7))
 (via (at 143.5 108) (size 0.6) (drill 0.3) (layers "F.Cu" "B.Cu") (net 7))
 (via (at 142.5 86) (size 0.6) (drill 0.3) (layers "F.Cu" "B.Cu") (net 7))
 (segment (start 142.5 107) (end 143.5 108) (width 0.2) (layer "B.Cu") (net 7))
 (segment (start 142.5 86) (end 142.5 107) (width 0.2) (layer "B.Cu") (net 7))
 (segment (start 142.2 108.2) (end 142.2 118.485) (width 0.2) (layer "F.Cu") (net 2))
 (segment (start 135.15 79) (end 135.15 85.4375) (width 0.2) (layer "F.Cu") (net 2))
 (segment (start 135.15 85.4375) (end 135 85.5875) (width 0.2) (layer "F.Cu") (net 2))
 (segment (start 135.9125 85.5875) (end 136.5 85) (width 0.2) (layer "F.Cu") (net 2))
 (segment (start 135 85.5875) (end 135.9125 85.5875) (width 0.2) (layer "F.Cu") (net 2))
 (segment (start 142 108) (end 142.2 108.2) (width 0.2) (layer "F.Cu") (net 2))
 (via (at 142 108) (size 0.6) (drill 0.3) (layers "F.Cu" "B.Cu") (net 2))
 (via (at 136.5 85) (size 0.6) (drill 0.3) (layers "F.Cu" "B.Cu") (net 2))
 (segment (start 141 107) (end 142 108) (width 0.2) (layer "B.Cu") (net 2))
 (segment (start 141 86) (end 141 107) (width 0.2) (layer "B.Cu") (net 2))
 (segment (start 136.5 85) (end 140 85) (width 0.2) (layer "B.Cu") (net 2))
 (segment (start 140 85) (end 141 86) (width 0.2) (layer "B.Cu") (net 2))
 (segment (start 141 85.5875) (end 139.9125 85.5875) (width 0.2) (layer "F.Cu") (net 10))
 (segment (start 140.23 84.8175) (end 141 85.5875) (width 0.2) (layer "F.Cu") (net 10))
 (segment (start 139.9125 85.5875) (end 139.5 86) (width 0.2) (layer "F.Cu") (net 10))
 (segment (start 140 108) (end 140 118.485) (width 0.2) (layer "F.Cu") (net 10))
 (segment (start 140.23 79) (end 140.23 84.8175) (width 0.2) (layer "F.Cu") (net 10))
 (via (at 139.5 86) (size 0.6) (drill 0.3) (layers "F.Cu" "B.Cu") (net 10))
 (via (at 140 108) (size 0.6) (drill 0.3) (layers "F.Cu" "B.Cu") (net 10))
 (segment (start 139.5 86) (end 139.5 107.5) (width 0.2) (layer "B.Cu") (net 10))
 (segment (start 139.5 107.5) (end 140 108) (width 0.2) (layer "B.Cu") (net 10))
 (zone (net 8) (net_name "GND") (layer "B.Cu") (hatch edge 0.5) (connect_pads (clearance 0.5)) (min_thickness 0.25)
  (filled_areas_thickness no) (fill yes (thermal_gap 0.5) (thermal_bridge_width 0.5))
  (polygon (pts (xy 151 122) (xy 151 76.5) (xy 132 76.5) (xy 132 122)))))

